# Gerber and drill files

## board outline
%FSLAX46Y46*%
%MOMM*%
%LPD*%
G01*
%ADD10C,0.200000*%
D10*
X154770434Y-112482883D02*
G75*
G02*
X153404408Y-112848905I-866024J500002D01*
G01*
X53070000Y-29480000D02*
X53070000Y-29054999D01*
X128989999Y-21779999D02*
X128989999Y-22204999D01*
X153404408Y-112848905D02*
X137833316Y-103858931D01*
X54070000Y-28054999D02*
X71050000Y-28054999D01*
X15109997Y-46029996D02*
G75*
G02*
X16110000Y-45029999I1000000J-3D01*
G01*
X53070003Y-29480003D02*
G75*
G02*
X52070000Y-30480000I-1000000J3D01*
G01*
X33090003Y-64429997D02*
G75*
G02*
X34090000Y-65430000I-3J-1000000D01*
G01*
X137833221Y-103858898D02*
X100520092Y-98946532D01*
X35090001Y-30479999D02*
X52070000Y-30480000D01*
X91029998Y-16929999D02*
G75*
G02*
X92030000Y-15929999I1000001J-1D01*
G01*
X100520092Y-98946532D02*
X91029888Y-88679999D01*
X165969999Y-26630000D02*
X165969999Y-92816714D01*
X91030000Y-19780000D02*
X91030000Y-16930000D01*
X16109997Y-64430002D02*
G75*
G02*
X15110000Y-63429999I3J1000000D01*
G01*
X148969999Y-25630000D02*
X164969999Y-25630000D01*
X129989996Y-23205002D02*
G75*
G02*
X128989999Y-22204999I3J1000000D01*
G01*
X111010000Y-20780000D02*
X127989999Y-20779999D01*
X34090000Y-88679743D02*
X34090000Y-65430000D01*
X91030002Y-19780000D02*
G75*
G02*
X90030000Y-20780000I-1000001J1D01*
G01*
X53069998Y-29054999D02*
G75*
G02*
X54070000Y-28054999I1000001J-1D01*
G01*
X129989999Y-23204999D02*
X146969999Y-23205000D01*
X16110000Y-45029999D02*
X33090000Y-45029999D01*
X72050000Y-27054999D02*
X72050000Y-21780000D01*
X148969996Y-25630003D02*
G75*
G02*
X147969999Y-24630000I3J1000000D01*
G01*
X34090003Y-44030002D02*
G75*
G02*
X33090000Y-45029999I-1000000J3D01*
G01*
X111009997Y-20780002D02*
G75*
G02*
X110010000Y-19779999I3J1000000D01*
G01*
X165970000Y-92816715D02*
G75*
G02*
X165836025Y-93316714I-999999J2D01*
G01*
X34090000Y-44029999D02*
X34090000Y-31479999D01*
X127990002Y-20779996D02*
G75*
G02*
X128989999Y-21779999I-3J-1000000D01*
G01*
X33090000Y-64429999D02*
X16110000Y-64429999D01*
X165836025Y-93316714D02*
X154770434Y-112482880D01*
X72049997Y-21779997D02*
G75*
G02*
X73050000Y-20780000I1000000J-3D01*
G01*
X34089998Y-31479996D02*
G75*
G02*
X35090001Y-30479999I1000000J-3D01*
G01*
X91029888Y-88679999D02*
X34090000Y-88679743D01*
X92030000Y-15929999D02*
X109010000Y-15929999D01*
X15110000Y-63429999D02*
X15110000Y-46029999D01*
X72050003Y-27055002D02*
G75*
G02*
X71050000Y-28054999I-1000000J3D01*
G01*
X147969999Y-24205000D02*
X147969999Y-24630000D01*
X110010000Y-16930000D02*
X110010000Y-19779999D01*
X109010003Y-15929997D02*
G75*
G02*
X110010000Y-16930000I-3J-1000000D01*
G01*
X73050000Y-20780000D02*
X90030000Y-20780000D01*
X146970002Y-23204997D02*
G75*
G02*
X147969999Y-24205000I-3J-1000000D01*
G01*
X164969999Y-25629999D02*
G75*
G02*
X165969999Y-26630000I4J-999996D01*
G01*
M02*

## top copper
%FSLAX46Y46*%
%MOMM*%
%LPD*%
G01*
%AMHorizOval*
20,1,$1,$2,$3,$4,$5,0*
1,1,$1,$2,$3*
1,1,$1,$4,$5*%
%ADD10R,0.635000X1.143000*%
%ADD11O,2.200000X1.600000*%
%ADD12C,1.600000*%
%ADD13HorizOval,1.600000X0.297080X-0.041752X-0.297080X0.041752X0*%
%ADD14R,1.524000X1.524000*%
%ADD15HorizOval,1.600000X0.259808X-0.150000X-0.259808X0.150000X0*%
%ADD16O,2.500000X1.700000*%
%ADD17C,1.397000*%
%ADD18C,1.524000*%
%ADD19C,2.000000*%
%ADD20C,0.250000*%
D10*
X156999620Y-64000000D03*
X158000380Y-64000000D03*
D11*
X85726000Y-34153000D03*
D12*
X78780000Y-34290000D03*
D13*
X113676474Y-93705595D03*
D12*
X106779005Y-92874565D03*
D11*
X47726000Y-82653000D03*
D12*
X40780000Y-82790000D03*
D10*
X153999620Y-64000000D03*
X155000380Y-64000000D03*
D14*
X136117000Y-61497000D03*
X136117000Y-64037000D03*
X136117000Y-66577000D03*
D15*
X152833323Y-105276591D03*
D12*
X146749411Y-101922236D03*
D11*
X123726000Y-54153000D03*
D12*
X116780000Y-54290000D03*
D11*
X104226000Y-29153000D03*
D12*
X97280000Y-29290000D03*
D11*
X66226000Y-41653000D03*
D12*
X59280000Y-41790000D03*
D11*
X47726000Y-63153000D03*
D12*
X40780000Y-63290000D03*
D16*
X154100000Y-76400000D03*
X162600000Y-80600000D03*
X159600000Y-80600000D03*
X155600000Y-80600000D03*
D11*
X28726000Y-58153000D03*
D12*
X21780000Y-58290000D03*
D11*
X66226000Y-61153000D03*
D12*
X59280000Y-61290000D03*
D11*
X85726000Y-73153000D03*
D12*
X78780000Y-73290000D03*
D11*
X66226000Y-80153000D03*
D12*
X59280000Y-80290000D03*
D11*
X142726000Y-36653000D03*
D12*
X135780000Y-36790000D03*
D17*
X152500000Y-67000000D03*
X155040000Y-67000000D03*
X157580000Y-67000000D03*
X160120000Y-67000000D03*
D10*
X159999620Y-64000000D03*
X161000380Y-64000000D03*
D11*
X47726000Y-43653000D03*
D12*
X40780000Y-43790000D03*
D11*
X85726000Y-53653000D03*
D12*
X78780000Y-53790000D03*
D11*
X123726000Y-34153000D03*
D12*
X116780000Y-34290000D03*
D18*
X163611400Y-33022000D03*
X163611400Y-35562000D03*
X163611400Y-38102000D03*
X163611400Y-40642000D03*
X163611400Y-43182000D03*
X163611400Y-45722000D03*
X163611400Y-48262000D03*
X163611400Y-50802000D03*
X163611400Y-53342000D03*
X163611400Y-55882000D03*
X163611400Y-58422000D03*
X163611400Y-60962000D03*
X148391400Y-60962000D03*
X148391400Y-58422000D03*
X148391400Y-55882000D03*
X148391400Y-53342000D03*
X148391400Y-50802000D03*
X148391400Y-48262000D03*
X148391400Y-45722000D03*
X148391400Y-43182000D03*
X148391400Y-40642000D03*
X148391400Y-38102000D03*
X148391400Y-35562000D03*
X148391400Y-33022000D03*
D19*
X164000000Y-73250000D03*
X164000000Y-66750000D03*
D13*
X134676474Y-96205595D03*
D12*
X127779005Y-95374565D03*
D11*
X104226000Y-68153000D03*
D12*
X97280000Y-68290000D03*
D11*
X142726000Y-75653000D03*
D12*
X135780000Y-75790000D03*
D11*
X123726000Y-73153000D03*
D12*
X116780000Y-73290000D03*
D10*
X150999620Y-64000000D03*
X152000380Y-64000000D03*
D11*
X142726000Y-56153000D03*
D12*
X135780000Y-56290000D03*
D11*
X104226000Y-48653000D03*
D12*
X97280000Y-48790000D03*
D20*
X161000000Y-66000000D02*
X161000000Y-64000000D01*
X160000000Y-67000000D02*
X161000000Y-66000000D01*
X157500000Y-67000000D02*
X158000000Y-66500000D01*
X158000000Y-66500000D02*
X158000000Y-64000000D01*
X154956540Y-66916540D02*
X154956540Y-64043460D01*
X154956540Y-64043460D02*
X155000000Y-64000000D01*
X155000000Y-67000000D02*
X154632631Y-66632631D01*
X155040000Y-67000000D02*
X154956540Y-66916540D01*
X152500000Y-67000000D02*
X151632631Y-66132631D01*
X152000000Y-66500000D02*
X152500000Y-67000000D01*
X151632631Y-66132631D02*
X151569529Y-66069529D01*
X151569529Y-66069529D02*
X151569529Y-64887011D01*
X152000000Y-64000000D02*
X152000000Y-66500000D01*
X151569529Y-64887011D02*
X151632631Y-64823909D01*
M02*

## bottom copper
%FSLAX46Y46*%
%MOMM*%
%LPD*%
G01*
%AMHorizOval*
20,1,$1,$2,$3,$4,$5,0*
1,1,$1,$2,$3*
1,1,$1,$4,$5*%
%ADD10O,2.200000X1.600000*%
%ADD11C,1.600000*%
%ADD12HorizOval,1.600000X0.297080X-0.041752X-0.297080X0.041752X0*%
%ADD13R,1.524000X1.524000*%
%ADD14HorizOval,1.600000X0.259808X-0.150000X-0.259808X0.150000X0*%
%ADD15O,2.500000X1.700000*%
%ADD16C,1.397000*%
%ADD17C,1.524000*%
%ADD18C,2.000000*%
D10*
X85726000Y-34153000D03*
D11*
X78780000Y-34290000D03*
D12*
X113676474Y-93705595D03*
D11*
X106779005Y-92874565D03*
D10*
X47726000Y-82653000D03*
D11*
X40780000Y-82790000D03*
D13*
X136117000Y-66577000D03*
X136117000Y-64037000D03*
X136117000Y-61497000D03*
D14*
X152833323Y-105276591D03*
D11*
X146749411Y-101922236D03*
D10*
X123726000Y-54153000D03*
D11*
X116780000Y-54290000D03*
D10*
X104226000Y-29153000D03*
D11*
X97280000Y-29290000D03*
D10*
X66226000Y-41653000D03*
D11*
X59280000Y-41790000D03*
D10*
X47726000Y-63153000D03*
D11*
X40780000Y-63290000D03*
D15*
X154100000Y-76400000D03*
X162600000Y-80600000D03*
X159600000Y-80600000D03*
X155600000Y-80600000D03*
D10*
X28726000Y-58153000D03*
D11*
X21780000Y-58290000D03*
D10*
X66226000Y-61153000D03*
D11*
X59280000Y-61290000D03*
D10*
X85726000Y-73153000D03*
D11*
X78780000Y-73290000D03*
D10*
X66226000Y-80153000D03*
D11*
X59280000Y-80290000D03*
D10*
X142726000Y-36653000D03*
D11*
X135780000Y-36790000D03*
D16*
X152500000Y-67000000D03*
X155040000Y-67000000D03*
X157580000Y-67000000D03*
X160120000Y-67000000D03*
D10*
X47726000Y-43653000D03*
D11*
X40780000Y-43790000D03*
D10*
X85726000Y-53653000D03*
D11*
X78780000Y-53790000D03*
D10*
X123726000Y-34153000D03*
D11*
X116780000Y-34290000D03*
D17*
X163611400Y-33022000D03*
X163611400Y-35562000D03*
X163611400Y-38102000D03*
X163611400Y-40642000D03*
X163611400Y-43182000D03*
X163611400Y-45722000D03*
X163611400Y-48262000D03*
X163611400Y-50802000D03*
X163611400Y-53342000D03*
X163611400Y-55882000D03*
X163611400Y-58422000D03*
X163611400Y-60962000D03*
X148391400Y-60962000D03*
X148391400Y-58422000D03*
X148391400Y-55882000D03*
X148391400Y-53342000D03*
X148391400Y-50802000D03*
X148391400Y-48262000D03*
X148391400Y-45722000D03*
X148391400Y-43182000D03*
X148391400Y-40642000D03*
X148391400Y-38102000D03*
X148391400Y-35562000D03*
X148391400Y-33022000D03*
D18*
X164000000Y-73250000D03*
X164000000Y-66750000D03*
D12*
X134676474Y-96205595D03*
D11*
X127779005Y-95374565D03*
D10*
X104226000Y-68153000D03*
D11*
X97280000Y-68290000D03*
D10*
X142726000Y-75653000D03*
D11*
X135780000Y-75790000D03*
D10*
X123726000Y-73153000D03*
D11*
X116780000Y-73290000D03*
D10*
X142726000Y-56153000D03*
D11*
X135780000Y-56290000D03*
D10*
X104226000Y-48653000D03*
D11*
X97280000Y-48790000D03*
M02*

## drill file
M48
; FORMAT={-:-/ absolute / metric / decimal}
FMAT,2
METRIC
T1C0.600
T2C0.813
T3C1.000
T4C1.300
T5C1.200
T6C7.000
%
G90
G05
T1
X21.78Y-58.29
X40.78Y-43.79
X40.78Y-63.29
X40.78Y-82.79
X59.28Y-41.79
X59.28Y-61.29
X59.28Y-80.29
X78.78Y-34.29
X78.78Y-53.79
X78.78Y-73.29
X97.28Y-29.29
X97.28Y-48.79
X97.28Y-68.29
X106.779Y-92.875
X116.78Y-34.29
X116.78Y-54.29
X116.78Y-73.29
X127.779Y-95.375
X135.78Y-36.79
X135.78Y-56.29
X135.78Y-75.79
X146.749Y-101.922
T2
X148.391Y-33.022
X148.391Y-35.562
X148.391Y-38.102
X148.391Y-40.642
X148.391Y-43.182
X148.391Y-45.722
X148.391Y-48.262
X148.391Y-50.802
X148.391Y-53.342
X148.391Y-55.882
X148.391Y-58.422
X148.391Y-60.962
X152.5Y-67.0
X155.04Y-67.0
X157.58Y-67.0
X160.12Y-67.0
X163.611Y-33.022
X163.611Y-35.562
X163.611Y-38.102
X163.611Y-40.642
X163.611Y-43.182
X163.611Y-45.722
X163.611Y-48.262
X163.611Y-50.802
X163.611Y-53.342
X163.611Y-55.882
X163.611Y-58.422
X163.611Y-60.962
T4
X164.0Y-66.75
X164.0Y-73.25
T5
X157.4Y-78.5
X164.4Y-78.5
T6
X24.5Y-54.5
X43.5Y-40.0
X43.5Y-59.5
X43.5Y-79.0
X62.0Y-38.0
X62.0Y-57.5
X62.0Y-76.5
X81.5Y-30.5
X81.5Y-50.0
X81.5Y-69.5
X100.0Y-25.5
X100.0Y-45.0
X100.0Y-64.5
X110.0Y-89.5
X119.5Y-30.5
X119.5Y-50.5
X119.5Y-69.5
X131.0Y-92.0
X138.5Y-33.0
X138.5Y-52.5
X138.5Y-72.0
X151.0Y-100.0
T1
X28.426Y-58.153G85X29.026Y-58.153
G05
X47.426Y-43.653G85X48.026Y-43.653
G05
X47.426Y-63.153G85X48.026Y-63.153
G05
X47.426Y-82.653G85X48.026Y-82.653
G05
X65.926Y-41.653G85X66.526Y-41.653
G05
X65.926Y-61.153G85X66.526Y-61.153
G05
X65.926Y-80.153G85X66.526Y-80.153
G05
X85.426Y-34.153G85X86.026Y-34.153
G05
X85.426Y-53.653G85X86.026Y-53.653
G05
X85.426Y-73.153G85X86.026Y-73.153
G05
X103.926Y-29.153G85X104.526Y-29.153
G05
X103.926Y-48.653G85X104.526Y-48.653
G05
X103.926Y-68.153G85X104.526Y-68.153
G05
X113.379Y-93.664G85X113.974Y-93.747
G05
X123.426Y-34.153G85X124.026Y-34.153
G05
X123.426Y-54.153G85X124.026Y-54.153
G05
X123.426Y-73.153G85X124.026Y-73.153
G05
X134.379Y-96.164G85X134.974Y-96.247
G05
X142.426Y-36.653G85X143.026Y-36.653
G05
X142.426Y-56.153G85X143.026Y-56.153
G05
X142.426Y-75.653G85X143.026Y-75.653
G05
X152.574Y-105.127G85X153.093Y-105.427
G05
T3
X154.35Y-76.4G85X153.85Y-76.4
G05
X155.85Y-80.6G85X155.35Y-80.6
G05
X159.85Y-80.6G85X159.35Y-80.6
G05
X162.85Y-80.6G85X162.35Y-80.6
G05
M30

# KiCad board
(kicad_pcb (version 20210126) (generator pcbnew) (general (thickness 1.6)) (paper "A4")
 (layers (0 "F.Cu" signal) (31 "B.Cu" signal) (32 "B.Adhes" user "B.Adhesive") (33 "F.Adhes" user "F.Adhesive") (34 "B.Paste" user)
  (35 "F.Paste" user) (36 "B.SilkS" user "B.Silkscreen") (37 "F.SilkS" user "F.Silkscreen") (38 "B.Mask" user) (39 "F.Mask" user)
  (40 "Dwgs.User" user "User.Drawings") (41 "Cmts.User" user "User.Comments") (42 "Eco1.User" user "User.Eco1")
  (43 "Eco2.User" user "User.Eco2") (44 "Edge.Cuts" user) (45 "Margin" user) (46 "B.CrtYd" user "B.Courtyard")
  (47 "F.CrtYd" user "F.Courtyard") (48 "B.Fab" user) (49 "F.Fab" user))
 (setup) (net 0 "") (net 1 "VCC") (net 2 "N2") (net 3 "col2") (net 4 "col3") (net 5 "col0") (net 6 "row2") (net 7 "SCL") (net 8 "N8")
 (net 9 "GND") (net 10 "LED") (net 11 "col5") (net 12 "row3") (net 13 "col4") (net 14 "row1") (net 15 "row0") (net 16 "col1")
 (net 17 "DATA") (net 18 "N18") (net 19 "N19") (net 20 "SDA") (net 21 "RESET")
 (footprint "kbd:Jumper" (layer "F.Cu") (at 157.5 64)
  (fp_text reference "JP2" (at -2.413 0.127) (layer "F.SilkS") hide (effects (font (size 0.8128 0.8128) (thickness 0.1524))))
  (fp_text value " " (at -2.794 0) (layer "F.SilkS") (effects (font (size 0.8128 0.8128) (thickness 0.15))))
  (pad "1" smd rect (at -0.50038 0) (locked) (size 0.635 1.143) (layers "F.Cu" "F.Paste" "F.Mask") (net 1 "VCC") (clearance 0.1905))
  (pad "2" smd rect (at 0.50038 0) (locked) (size 0.635 1.143) (layers "F.Cu" "F.Paste" "F.Mask") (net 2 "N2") (clearance 0.1905)))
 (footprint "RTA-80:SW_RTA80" (layer "F.Cu") (at 81.5 30.5)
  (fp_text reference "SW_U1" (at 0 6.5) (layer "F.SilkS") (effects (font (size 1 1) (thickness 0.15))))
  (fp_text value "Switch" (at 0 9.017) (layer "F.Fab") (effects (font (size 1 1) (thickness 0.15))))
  (pad "" np_thru_hole circle (at 0 0) (locked) (size 7 7) (drill 7) (layers *.Cu *.Mask))
  (pad "1" thru_hole oval (at 4.226 3.653) (locked) (size 2.2 1.6) (drill oval 1.2 0.6) (layers *.Cu *.Mask) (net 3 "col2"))
  (pad "2" thru_hole circle (at -2.72 3.79) (locked) (size 1.6 1.6) (drill 0.6) (layers *.Cu *.Mask)))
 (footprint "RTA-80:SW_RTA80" (layer "F.Cu") (at 110 89.5 -8)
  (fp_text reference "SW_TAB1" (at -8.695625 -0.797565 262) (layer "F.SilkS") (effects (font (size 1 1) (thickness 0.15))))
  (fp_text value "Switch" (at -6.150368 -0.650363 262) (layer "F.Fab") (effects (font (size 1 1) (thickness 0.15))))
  (pad "" np_thru_hole circle (at 0 0 352) (locked) (size 7 7) (drill 7) (layers *.Cu *.Mask))
  (pad "1" thru_hole oval (at 4.226 3.653 352) (locked) (size 2.2 1.6) (drill oval 1.2 0.6) (layers *.Cu *.Mask) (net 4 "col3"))
  (pad "2" thru_hole circle (at -2.72 3.79 352) (locked) (size 1.6 1.6) (drill 0.6) (layers *.Cu *.Mask)))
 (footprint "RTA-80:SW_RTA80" (layer "F.Cu") (at 43.5 79)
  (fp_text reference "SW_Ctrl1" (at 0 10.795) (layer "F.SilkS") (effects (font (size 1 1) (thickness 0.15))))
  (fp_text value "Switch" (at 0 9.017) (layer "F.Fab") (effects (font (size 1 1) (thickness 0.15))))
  (pad "" np_thru_hole circle (at 0 0) (locked) (size 7 7) (drill 7) (layers *.Cu *.Mask))
  (pad "1" thru_hole oval (at 4.226 3.653) (locked) (size 2.2 1.6) (drill oval 1.2 0.6) (layers *.Cu *.Mask) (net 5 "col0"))
  (pad "2" thru_hole circle (at -2.72 3.79) (locked) (size 1.6 1.6) (drill 0.6) (layers *.Cu *.Mask) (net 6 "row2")))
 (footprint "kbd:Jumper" (layer "F.Cu") (at 154.5 64)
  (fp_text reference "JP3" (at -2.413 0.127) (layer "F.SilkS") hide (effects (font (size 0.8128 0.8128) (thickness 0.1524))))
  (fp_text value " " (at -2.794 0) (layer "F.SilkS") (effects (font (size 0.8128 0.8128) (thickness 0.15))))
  (pad "1" smd rect (at -0.50038 0) (locked) (size 0.635 1.143) (layers "F.Cu" "F.Paste" "F.Mask") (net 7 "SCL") (clearance 0.1905))
  (pad "2" smd rect (at 0.50038 0) (locked) (size 0.635 1.143) (layers "F.Cu" "F.Paste" "F.Mask") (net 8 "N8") (clearance 0.1905)))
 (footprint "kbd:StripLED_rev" (layer "F.Cu") (at 136.117 61.497)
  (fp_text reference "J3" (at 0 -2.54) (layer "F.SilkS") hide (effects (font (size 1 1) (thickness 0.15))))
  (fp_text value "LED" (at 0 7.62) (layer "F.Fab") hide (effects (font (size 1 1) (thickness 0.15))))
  (pad "1" smd rect (at 0 0) (locked) (size 1.524 1.524) (layers "F.Cu" "F.Paste" "F.Mask") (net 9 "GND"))
  (pad "1" smd rect (at 0 5.08) (locked) (size 1.524 1.524) (layers "B.Cu" "B.Paste" "B.Mask") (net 9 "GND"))
  (pad "2" smd rect (at 0 2.54) (locked) (size 1.524 1.524) (layers "B.Cu" "B.Paste" "B.Mask") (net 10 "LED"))
  (pad "2" smd rect (at 0 2.54) (locked) (size 1.524 1.524) (layers "F.Cu" "F.Paste" "F.Mask") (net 10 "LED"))
  (pad "3" smd rect (at 0 0) (locked) (size 1.524 1.524) (layers "B.Cu" "B.Paste" "B.Mask") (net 1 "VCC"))
  (pad "3" smd rect (at 0 5.08) (locked) (size 1.524 1.524) (layers "F.Cu" "F.Paste" "F.Mask") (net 1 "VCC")))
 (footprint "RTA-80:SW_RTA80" (layer "F.Cu") (at 151 100 -30)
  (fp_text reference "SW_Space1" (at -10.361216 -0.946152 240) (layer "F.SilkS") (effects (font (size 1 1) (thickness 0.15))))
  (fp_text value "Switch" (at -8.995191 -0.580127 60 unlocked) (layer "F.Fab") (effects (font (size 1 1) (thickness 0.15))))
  (pad "" np_thru_hole circle (at 0 0 330) (locked) (size 7 7) (drill 7) (layers *.Cu *.Mask))
  (pad "1" thru_hole oval (at 4.226 3.653 330) (locked) (size 2.2 1.6) (drill oval 1.2 0.6) (layers *.Cu *.Mask) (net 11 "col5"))
  (pad "2" thru_hole circle (at -2.72 3.79 330) (locked) (size 1.6 1.6) (drill 0.6) (layers *.Cu *.Mask) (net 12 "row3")))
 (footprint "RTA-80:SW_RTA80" (layer "F.Cu") (at 119.5 50.5)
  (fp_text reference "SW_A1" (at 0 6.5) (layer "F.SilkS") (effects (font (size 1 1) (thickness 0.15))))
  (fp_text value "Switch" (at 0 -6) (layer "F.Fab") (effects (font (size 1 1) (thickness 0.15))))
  (pad "" np_thru_hole circle (at 0 0) (locked) (size 7 7) (drill 7) (layers *.Cu *.Mask))
  (pad "1" thru_hole oval (at 4.226 3.653) (locked) (size 2.2 1.6) (drill oval 1.2 0.6) (layers *.Cu *.Mask) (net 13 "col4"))
  (pad "2" thru_hole circle (at -2.72 3.79) (locked) (size 1.6 1.6) (drill 0.6) (layers *.Cu *.Mask) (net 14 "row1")))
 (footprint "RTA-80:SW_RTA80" (layer "F.Cu") (at 100 25.5)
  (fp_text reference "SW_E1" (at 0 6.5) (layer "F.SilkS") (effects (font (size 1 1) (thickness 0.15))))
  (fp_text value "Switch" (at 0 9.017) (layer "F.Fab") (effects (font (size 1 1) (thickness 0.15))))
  (pad "" np_thru_hole circle (at 0 0) (locked) (size 7 7) (drill 7) (layers *.Cu *.Mask))
  (pad "1" thru_hole oval (at 4.226 3.653) (locked) (size 2.2 1.6) (drill oval 1.2 0.6) (layers *.Cu *.Mask) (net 4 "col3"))
  (pad "2" thru_hole circle (at -2.72 3.79) (locked) (size 1.6 1.6) (drill 0.6) (layers *.Cu *.Mask) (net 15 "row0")))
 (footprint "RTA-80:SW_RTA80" (layer "F.Cu") (at 62 38)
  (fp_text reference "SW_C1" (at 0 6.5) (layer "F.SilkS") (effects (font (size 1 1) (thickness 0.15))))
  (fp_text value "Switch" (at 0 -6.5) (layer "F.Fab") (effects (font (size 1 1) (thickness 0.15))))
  (pad "" np_thru_hole circle (at 0 0) (locked) (size 7 7) (drill 7) (layers *.Cu *.Mask))
  (pad "1" thru_hole oval (at 4.226 3.653) (locked) (size 2.2 1.6) (drill oval 1.2 0.6) (layers *.Cu *.Mask) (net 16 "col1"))
  (pad "2" thru_hole circle (at -2.72 3.79) (locked) (size 1.6 1.6) (drill 0.6) (layers *.Cu *.Mask) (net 15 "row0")))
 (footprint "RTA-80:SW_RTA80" (layer "F.Cu") (at 43.5 59.5)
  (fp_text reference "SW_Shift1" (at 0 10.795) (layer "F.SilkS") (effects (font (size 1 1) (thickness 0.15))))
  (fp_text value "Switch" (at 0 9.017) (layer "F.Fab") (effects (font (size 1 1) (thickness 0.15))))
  (pad "" np_thru_hole circle (at 0 0) (locked) (size 7 7) (drill 7) (layers *.Cu *.Mask))
  (pad "1" thru_hole oval (at 4.226 3.653) (locked) (size 2.2 1.6) (drill oval 1.2 0.6) (layers *.Cu *.Mask) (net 5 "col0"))
  (pad "2" thru_hole circle (at -2.72 3.79) (locked) (size 1.6 1.6) (drill 0.6) (layers *.Cu *.Mask) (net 14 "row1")))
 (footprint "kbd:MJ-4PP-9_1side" (layer "F.Cu") (at 165.9 78.5 -90)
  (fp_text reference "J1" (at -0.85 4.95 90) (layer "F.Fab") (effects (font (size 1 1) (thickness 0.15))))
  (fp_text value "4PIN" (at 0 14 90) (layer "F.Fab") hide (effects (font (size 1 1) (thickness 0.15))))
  (pad "" np_thru_hole circle (at 0 8.5 270) (locked) (size 1.2 1.2) (drill 1.2) (layers *.Cu *.Mask))
  (pad "" np_thru_hole circle (at 0 1.5 270) (locked) (size 1.2 1.2) (drill 1.2) (layers *.Cu *.Mask))
  (pad "A" thru_hole oval (at -2.1 11.8 270) (locked) (size 1.7 2.5) (drill oval 1 1.5) (layers *.Cu "B.Mask") (clearance 0.15))
  (pad "B" thru_hole oval (at 2.1 3.3 270) (locked) (size 1.7 2.5) (drill oval 1 1.5) (layers *.Cu "B.Mask") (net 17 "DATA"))
  (pad "C" thru_hole oval (at 2.1 6.3 270) (locked) (size 1.7 2.5) (drill oval 1 1.5) (layers *.Cu "B.Mask") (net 9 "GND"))
  (pad "D" thru_hole oval (at 2.1 10.3 270) (locked) (size 1.7 2.5) (drill oval 1 1.5) (layers *.Cu "B.Mask") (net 1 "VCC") (clearance 0.15)))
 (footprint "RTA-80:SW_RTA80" (layer "F.Cu") (at 24.5 54.5)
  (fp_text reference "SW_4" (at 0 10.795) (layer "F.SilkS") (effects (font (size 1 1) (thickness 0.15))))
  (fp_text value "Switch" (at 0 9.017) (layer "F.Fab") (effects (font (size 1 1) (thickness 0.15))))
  (pad "" np_thru_hole circle (at 0 0) (locked) (size 7 7) (drill 7) (layers *.Cu *.Mask))
  (pad "1" thru_hole oval (at 4.226 3.653) (locked) (size 2.2 1.6) (drill oval 1.2 0.6) (layers *.Cu *.Mask) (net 5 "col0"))
  (pad "2" thru_hole circle (at -2.72 3.79) (locked) (size 1.6 1.6) (drill 0.6) (layers *.Cu *.Mask) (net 12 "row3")))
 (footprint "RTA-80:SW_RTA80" (layer "F.Cu") (at 62 57.5)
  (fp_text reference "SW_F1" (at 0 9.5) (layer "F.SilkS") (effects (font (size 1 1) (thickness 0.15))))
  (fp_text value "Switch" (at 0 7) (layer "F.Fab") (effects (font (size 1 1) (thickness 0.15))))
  (pad "" np_thru_hole circle (at 0 0) (locked) (size 7 7) (drill 7) (layers *.Cu *.Mask))
  (pad "1" thru_hole oval (at 4.226 3.653) (locked) (size 2.2 1.6) (drill oval 1.2 0.6) (layers *.Cu *.Mask) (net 16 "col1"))
  (pad "2" thru_hole circle (at -2.72 3.79) (locked) (size 1.6 1.6) (drill 0.6) (layers *.Cu *.Mask) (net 14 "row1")))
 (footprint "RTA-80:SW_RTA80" (layer "F.Cu") (at 81.5 69.5)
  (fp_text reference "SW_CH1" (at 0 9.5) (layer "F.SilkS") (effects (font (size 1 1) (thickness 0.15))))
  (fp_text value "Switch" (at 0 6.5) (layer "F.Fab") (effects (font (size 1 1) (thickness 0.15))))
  (pad "" np_thru_hole circle (at 0 0) (locked) (size 7 7) (drill 7) (layers *.Cu *.Mask))
  (pad "1" thru_hole oval (at 4.226 3.653) (locked) (size 2.2 1.6) (drill oval 1.2 0.6) (layers *.Cu *.Mask) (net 3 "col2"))
  (pad "2" thru_hole circle (at -2.72 3.79) (locked) (size 1.6 1.6) (drill 0.6) (layers *.Cu *.Mask) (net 6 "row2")))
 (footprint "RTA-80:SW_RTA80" (layer "F.Cu") (at 62 76.5)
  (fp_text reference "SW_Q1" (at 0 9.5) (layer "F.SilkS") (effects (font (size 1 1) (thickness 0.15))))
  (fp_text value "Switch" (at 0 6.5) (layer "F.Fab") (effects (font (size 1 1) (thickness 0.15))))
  (pad "" np_thru_hole circle (at 0 0) (locked) (size 7 7) (drill 7) (layers *.Cu *.Mask))
  (pad "1" thru_hole oval (at 4.226 3.653) (locked) (size 2.2 1.6) (drill oval 1.2 0.6) (layers *.Cu *.Mask) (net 16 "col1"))
  (pad "2" thru_hole circle (at -2.72 3.79) (locked) (size 1.6 1.6) (drill 0.6) (layers *.Cu *.Mask) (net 6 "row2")))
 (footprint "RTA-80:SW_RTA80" (layer "F.Cu") (at 138.5 33)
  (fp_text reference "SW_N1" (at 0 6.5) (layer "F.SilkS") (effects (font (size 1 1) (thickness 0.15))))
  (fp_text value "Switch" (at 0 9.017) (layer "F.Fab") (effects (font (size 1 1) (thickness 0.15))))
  (pad "" np_thru_hole circle (at 0 0) (locked) (size 7 7) (drill 7) (layers *.Cu *.Mask))
  (pad "1" thru_hole oval (at 4.226 3.653) (locked) (size 2.2 1.6) (drill oval 1.2 0.6) (layers *.Cu *.Mask) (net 11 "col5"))
  (pad "2" thru_hole circle (at -2.72 3.79) (locked) (size 1.6 1.6) (drill 0.6) (layers *.Cu *.Mask) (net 15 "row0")))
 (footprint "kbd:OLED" (layer "F.Cu") (at 152.5 67)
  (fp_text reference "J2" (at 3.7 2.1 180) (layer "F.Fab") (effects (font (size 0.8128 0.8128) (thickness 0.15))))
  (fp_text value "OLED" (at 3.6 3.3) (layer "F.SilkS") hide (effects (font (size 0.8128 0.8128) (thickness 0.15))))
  (pad "1" thru_hole circle (at 0 0) (locked) (size 1.397 1.397) (drill 0.8128) (layers *.Cu *.Mask "F.SilkS") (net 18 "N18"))
  (pad "2" thru_hole circle (at 2.54 0) (locked) (size 1.397 1.397) (drill 0.8128) (layers *.Cu *.Mask "F.SilkS") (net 8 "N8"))
  (pad "3" thru_hole circle (at 5.08 0) (locked) (size 1.397 1.397) (drill 0.8128) (layers *.Cu *.Mask "F.SilkS") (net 2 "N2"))
  (pad "4" thru_hole circle (at 7.62 0) (locked) (size 1.397 1.397) (drill 0.8128) (layers *.Cu *.Mask "F.SilkS") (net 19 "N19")))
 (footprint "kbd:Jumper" (layer "F.Cu") (at 160.5 64)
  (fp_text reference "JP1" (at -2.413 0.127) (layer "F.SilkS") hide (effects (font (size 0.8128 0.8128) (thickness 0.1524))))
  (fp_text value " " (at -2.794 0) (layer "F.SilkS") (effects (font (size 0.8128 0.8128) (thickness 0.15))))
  (pad "1" smd rect (at -0.50038 0) (locked) (size 0.635 1.143) (layers "F.Cu" "F.Paste" "F.Mask") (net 9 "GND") (clearance 0.1905))
  (pad "2" smd rect (at 0.50038 0) (locked) (size 0.635 1.143) (layers "F.Cu" "F.Paste" "F.Mask") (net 19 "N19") (clearance 0.1905)))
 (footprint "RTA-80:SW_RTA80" (layer "F.Cu") (at 43.5 40)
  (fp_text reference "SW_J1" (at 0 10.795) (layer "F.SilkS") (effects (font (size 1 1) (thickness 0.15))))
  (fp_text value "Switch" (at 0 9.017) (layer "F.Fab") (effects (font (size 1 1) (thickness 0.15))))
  (pad "" np_thru_hole circle (at 0 0) (locked) (size 7 7) (drill 7) (layers *.Cu *.Mask))
  (pad "1" thru_hole oval (at 4.226 3.653) (locked) (size 2.2 1.6) (drill oval 1.2 0.6) (layers *.Cu *.Mask) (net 5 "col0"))
  (pad "2" thru_hole circle (at -2.72 3.79) (locked) (size 1.6 1.6) (drill 0.6) (layers *.Cu *.Mask) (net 15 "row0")))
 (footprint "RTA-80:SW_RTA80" (layer "F.Cu") (at 81.5 50)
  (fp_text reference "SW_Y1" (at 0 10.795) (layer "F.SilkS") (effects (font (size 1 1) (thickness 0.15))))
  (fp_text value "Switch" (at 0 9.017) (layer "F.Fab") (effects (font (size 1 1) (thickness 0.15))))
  (pad "" np_thru_hole circle (at 0 0) (locked) (size 7 7) (drill 7) (layers *.Cu *.Mask))
  (pad "1" thru_hole oval (at 4.226 3.653) (locked) (size 2.2 1.6) (drill oval 1.2 0.6) (layers *.Cu *.Mask) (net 3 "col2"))
  (pad "2" thru_hole circle (at -2.72 3.79) (locked) (size 1.6 1.6) (drill 0.6) (layers *.Cu *.Mask) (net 14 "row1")))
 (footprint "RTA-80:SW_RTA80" (layer "F.Cu") (at 119.5 30.5)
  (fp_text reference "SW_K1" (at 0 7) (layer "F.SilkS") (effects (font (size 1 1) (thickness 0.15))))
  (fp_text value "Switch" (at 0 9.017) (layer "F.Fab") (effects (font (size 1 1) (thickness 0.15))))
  (pad "" np_thru_hole circle (at 0 0) (locked) (size 7 7) (drill 7) (layers *.Cu *.Mask))
  (pad "1" thru_hole oval (at 4.226 3.653) (locked) (size 2.2 1.6) (drill oval 1.2 0.6) (layers *.Cu *.Mask) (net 13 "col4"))
  (pad "2" thru_hole circle (at -2.72 3.79) (locked) (size 1.6 1.6) (drill 0.6) (layers *.Cu *.Mask)))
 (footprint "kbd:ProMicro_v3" (layer "F.Cu") (at 156 47.5)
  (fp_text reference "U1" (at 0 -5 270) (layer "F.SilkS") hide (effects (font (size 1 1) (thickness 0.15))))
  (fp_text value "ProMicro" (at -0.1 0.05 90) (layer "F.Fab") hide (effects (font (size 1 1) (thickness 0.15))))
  (pad "1" thru_hole circle (at 7.6114 -14.478) (locked) (size 1.524 1.524) (drill 0.8128) (layers *.Cu "B.Mask") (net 10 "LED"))
  (pad "2" thru_hole circle (at 7.6114 -11.938) (locked) (size 1.524 1.524) (drill 0.8128) (layers *.Cu "B.Mask") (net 17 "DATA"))
  (pad "3" thru_hole circle (at 7.6114 -9.398) (locked) (size 1.524 1.524) (drill 0.8128) (layers *.Cu "B.Mask") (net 9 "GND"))
  (pad "4" thru_hole circle (at 7.6114 -6.858) (locked) (size 1.524 1.524) (drill 0.8128) (layers *.Cu "B.Mask") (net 9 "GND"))
  (pad "5" thru_hole circle (at 7.6114 -4.318) (locked) (size 1.524 1.524) (drill 0.8128) (layers *.Cu "B.Mask") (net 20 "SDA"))
  (pad "6" thru_hole circle (at 7.6114 -1.778) (locked) (size 1.524 1.524) (drill 0.8128) (layers *.Cu "B.Mask") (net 7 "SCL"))
  (pad "7" thru_hole circle (at 7.6114 0.762) (locked) (size 1.524 1.524) (drill 0.8128) (layers *.Cu "B.Mask"))
  (pad "8" thru_hole circle (at 7.6114 3.302) (locked) (size 1.524 1.524) (drill 0.8128) (layers *.Cu "B.Mask") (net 15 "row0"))
  (pad "9" thru_hole circle (at 7.6114 5.842) (locked) (size 1.524 1.524) (drill 0.8128) (layers *.Cu "B.Mask") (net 14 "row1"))
  (pad "10" thru_hole circle (at 7.6114 8.382) (locked) (size 1.524 1.524) (drill 0.8128) (layers *.Cu "B.Mask") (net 6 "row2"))
  (pad "11" thru_hole circle (at 7.6114 10.922) (locked) (size 1.524 1.524) (drill 0.8128) (layers *.Cu "B.Mask") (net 12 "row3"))
  (pad "12" thru_hole circle (at 7.6114 13.462) (locked) (size 1.524 1.524) (drill 0.8128) (layers *.Cu "B.Mask"))
  (pad "13" thru_hole circle (at -7.6086 13.462) (locked) (size 1.524 1.524) (drill 0.8128) (layers *.Cu "B.Mask") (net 11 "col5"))
  (pad "14" thru_hole circle (at -7.6086 10.922) (locked) (size 1.524 1.524) (drill 0.8128) (layers *.Cu "B.Mask") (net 13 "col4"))
  (pad "15" thru_hole circle (at -7.6086 8.382) (locked) (size 1.524 1.524) (drill 0.8128) (layers *.Cu "B.Mask") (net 4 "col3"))
  (pad "16" thru_hole circle (at -7.6086 5.842) (locked) (size 1.524 1.524) (drill 0.8128) (layers *.Cu "B.Mask") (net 3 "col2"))
  (pad "17" thru_hole circle (at -7.6086 3.302) (locked) (size 1.524 1.524) (drill 0.8128) (layers *.Cu "B.Mask") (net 16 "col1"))
  (pad "18" thru_hole circle (at -7.6086 0.762) (locked) (size 1.524 1.524) (drill 0.8128) (layers *.Cu "B.Mask") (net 5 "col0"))
  (pad "19" thru_hole circle (at -7.6086 -1.778) (locked) (size 1.524 1.524) (drill 0.8128) (layers *.Cu "B.Mask"))
  (pad "20" thru_hole circle (at -7.6086 -4.318) (locked) (size 1.524 1.524) (drill 0.8128) (layers *.Cu "B.Mask"))
  (pad "21" thru_hole circle (at -7.6086 -6.858) (locked) (size 1.524 1.524) (drill 0.8128) (layers *.Cu "B.Mask") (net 1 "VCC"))
  (pad "22" thru_hole circle (at -7.6086 -9.398) (locked) (size 1.524 1.524) (drill 0.8128) (layers *.Cu "B.Mask") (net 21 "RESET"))
  (pad "23" thru_hole circle (at -7.6086 -11.938) (locked) (size 1.524 1.524) (drill 0.8128) (layers *.Cu "B.Mask") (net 9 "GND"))
  (pad "24" thru_hole circle (at -7.6086 -14.478) (locked) (size 1.524 1.524) (drill 0.8128) (layers *.Cu "B.Mask")))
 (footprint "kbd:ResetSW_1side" (layer "F.Cu") (at 164 70 -90)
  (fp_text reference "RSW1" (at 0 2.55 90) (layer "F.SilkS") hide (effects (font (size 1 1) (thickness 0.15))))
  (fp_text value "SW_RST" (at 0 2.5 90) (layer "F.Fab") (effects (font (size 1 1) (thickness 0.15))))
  (pad "1" thru_hole circle (at 3.25 0 270) (locked) (size 2 2) (drill 1.3) (layers *.Cu "B.Mask") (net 9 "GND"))
  (pad "2" thru_hole circle (at -3.25 0 270) (locked) (size 2 2) (drill 1.3) (layers *.Cu "B.Mask") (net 21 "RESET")))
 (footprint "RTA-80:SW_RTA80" (layer "F.Cu") (at 131 92 -8)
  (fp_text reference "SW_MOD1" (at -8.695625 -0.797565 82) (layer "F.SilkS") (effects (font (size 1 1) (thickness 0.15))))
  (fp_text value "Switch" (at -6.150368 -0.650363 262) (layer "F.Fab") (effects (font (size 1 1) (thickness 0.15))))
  (pad "" np_thru_hole circle (at 0 0 352) (locked) (size 7 7) (drill 7) (layers *.Cu *.Mask))
  (pad "1" thru_hole oval (at 4.226 3.653 352) (locked) (size 2.2 1.6) (drill oval 1.2 0.6) (layers *.Cu *.Mask) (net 13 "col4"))
  (pad "2" thru_hole circle (at -2.72 3.79 352) (locked) (size 1.6 1.6) (drill 0.6) (layers *.Cu *.Mask) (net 12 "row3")))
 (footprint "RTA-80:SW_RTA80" (layer "F.Cu") (at 100 64.5)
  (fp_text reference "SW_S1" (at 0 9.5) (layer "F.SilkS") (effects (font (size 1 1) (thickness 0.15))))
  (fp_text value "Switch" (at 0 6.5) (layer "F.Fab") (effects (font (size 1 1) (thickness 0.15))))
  (pad "" np_thru_hole circle (at 0 0) (locked) (size 7 7) (drill 7) (layers *.Cu *.Mask))
  (pad "1" thru_hole oval (at 4.226 3.653) (locked) (size 2.2 1.6) (drill oval 1.2 0.6) (layers *.Cu *.Mask) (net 4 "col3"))
  (pad "2" thru_hole circle (at -2.72 3.79) (locked) (size 1.6 1.6) (drill 0.6) (layers *.Cu *.Mask)))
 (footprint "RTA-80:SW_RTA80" (layer "F.Cu") (at 138.5 72)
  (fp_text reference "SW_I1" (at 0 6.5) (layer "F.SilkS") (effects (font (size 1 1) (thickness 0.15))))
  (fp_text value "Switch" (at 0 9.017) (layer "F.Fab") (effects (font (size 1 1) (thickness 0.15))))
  (pad "" np_thru_hole circle (at 0 0) (locked) (size 7 7) (drill 7) (layers *.Cu *.Mask))
  (pad "1" thru_hole oval (at 4.226 3.653) (locked) (size 2.2 1.6) (drill oval 1.2 0.6) (layers *.Cu *.Mask) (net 11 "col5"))
  (pad "2" thru_hole circle (at -2.72 3.79) (locked) (size 1.6 1.6) (drill 0.6) (layers *.Cu *.Mask) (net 6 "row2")))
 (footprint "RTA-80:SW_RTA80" (layer "F.Cu") (at 119.5 69.5)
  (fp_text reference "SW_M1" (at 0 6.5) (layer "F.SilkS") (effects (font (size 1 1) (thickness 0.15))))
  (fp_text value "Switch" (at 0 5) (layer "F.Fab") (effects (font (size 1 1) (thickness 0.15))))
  (pad "" np_thru_hole circle (at 0 0) (locked) (size 7 7) (drill 7) (layers *.Cu *.Mask))
  (pad "1" thru_hole oval (at 4.226 3.653) (locked) (size 2.2 1.6) (drill oval 1.2 0.6) (layers *.Cu *.Mask) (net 13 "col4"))
  (pad "2" thru_hole circle (at -2.72 3.79) (locked) (size 1.6 1.6) (drill 0.6) (layers *.Cu *.Mask) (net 6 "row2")))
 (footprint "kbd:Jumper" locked (layer "F.Cu") (at 151.5 64)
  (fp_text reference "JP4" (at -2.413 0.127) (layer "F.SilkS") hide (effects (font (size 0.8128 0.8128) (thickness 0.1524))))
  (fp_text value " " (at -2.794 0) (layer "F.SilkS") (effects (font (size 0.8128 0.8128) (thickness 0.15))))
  (pad "1" smd rect (at -0.50038 0) (locked) (size 0.635 1.143) (layers "F.Cu" "F.Paste" "F.Mask") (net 20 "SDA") (clearance 0.1905))
  (pad "2" smd rect (at 0.50038 0) (locked) (size 0.635 1.143) (layers "F.Cu" "F.Paste" "F.Mask") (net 18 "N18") (clearance 0.1905)))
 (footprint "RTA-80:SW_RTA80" (layer "F.Cu") (at 138.5 52.5)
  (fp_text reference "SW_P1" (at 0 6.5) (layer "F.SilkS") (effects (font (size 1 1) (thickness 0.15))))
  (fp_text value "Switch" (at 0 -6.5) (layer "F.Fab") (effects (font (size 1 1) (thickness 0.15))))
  (pad "" np_thru_hole circle (at 0 0) (locked) (size 7 7) (drill 7) (layers *.Cu *.Mask))
  (pad "1" thru_hole oval (at 4.226 3.653) (locked) (size 2.2 1.6) (drill oval 1.2 0.6) (layers *.Cu *.Mask) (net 11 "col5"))
  (pad "2" thru_hole circle (at -2.72 3.79) (locked) (size 1.6 1.6) (drill 0.6) (layers *.Cu *.Mask) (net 14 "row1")))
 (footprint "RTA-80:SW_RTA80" (layer "F.Cu") (at 100 45)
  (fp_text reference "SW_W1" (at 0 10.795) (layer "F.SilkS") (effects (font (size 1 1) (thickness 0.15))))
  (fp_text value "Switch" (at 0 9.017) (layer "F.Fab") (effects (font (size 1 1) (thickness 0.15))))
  (pad "" np_thru_hole circle (at 0 0) (locked) (size 7 7) (drill 7) (layers *.Cu *.Mask))
  (pad "1" thru_hole oval (at 4.226 3.653) (locked) (size 2.2 1.6) (drill oval 1.2 0.6) (layers *.Cu *.Mask) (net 4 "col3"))
  (pad "2" thru_hole circle (at -2.72 3.79) (locked) (size 1.6 1.6) (drill 0.6) (layers *.Cu *.Mask)))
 (gr_arc (start 153.90441 111.982881) (end 153.404408 112.848905) (angle -90) (layer "Edge.Cuts") (width 0.2))
 (gr_line (start 53.07 29.48) (end 53.07 29.054999) (layer "Edge.Cuts") (width 0.2))
 (gr_line (start 128.989999 21.779999) (end 128.989999 22.204999) (layer "Edge.Cuts") (width 0.2))
 (gr_line (start 153.404408 112.848905) (end 137.833316 103.858931) (layer "Edge.Cuts") (width 0.2))
 (gr_line (start 54.07 28.054999) (end 71.05 28.054999) (layer "Edge.Cuts") (width 0.2))
 (gr_arc (start 16.109997 46.029999) (end 16.11 45.029999) (angle -90) (layer "Edge.Cuts") (width 0.2))
 (gr_arc (start 52.070003 29.48) (end 52.07 30.48) (angle -90) (layer "Edge.Cuts") (width 0.2))
 (gr_arc (start 33.09 65.429997) (end 34.09 65.43) (angle -90) (layer "Edge.Cuts") (width 0.2))
 (gr_line (start 137.833221 103.858898) (end 100.520092 98.946532) (layer "Edge.Cuts") (width 0.2))
 (gr_line (start 35.090001 30.479999) (end 52.07 30.48) (layer "Edge.Cuts") (width 0.2))
 (gr_arc (start 92.029999 16.93) (end 92.03 15.929999) (angle -90) (layer "Edge.Cuts") (width 0.2))
 (gr_line (start 100.520092 98.946532) (end 91.029888 88.679999) (layer "Edge.Cuts") (width 0.2))
 (gr_line (start 165.969999 26.63) (end 165.969999 92.816714) (layer "Edge.Cuts") (width 0.2))
 (gr_line (start 91.03 19.78) (end 91.03 16.93) (layer "Edge.Cuts") (width 0.2))
 (gr_arc (start 16.11 63.430002) (end 15.11 63.429999) (angle -90) (layer "Edge.Cuts") (width 0.2))
 (gr_line (start 148.969999 25.63) (end 164.969999 25.63) (layer "Edge.Cuts") (width 0.2))
 (gr_arc (start 129.989999 22.205002) (end 128.989999 22.204999) (angle -90) (layer "Edge.Cuts") (width 0.2))
 (gr_line (start 111.01 20.78) (end 127.989999 20.779999) (layer "Edge.Cuts") (width 0.2))
 (gr_line (start 34.09 88.679743) (end 34.09 65.43) (layer "Edge.Cuts") (width 0.2))
 (gr_arc (start 90.030001 19.779999) (end 90.03 20.78) (angle -90) (layer "Edge.Cuts") (width 0.2))
 (gr_arc (start 54.069999 29.055) (end 54.07 28.054999) (angle -90) (layer "Edge.Cuts") (width 0.2))
 (gr_line (start 129.989999 23.204999) (end 146.969999 23.205) (layer "Edge.Cuts") (width 0.2))
 (gr_line (start 16.11 45.029999) (end 33.09 45.029999) (layer "Edge.Cuts") (width 0.2))
 (gr_line (start 72.05 27.054999) (end 72.05 21.78) (layer "Edge.Cuts") (width 0.2))
 (gr_arc (start 148.969999 24.630003) (end 147.969999 24.63) (angle -90) (layer "Edge.Cuts") (width 0.2))
 (gr_arc (start 33.090003 44.029999) (end 33.09 45.029999) (angle -90) (layer "Edge.Cuts") (width 0.2))
 (gr_arc (start 111.01 19.780002) (end 110.01 19.779999) (angle -90) (layer "Edge.Cuts") (width 0.2))
 (gr_arc (start 164.970001 92.816713) (end 165.836025 93.316714) (angle -30) (layer "Edge.Cuts") (width 0.2))
 (gr_line (start 34.09 44.029999) (end 34.09 31.479999) (layer "Edge.Cuts") (width 0.2))
 (gr_arc (start 127.989999 21.779996) (end 128.989999 21.779999) (angle -90) (layer "Edge.Cuts") (width 0.2))
 (gr_line (start 33.09 64.429999) (end 16.11 64.429999) (layer "Edge.Cuts") (width 0.2))
 (gr_line (start 165.836025 93.316714) (end 154.770434 112.48288) (layer "Edge.Cuts") (width 0.2))
 (gr_arc (start 73.049997 21.78) (end 73.05 20.78) (angle -90) (layer "Edge.Cuts") (width 0.2))
 (gr_arc (start 35.089998 31.479999) (end 35.090001 30.479999) (angle -90) (layer "Edge.Cuts") (width 0.2))
 (gr_line (start 91.029888 88.679999) (end 34.09 88.679743) (layer "Edge.Cuts") (width 0.2))
 (gr_line (start 92.03 15.929999) (end 109.01 15.929999) (layer "Edge.Cuts") (width 0.2))
 (gr_line (start 15.11 63.429999) (end 15.11 46.029999) (layer "Edge.Cuts") (width 0.2))
 (gr_arc (start 71.050003 27.054999) (end 71.05 28.054999) (angle -90) (layer "Edge.Cuts") (width 0.2))
 (gr_line (start 147.969999 24.205) (end 147.969999 24.63) (layer "Edge.Cuts") (width 0.2))
 (gr_line (start 110.01 16.93) (end 110.01 19.779999) (layer "Edge.Cuts") (width 0.2))
 (gr_arc (start 109.01 16.929997) (end 110.01 16.93) (angle -90) (layer "Edge.Cuts") (width 0.2))
 (gr_line (start 73.05 20.78) (end 90.03 20.78) (layer "Edge.Cuts") (width 0.2))
 (gr_arc (start 146.969999 24.204997) (end 147.969999 24.205) (angle -90) (layer "Edge.Cuts") (width 0.2))
 (gr_arc (start 164.970003 26.629995) (end 165.969999 26.63) (angle -90.00051566) (layer "Edge.Cuts") (width 0.2))
 (segment (start 161 66) (end 161 64) (width 0.25) (layer "F.Cu") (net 19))
 (segment (start 160 67) (end 161 66) (width 0.25) (layer "F.Cu") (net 19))
 (segment (start 157.5 67) (end 158 66.5) (width 0.25) (layer "F.Cu") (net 2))
 (segment (start 158 66.5) (end 158 64) (width 0.25) (layer "F.Cu") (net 2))
 (segment (start 154.95654 66.91654) (end 154.95654 64.04346) (width 0.25) (layer "F.Cu") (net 8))
 (segment (start 154.95654 64.04346) (end 155 64) (width 0.25) (layer "F.Cu") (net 8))
 (segment (start 155 67) (end 154.632631 66.632631) (width 0.25) (layer "F.Cu") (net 8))
 (segment (start 155.04 67) (end 154.95654 66.91654) (width 0.25) (layer "F.Cu") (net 8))
 (segment (start 152.5 67) (end 151.632631 66.132631) (width 0.25) (layer "F.Cu") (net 18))
 (segment (start 152 66.5) (end 152.5 67) (width 0.25) (layer "F.Cu") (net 18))
 (segment (start 151.632631 66.132631) (end 151.569529 66.069529) (width 0.25) (layer "F.Cu") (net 18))
 (segment (start 151.569529 66.069529) (end 151.569529 64.887011) (width 0.25) (layer "F.Cu") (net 18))
 (segment (start 152 64) (end 152 66.5) (width 0.25) (layer "F.Cu") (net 18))
 (segment (start 151.569529 64.887011) (end 151.632631 64.823909) (width 0.25) (layer "F.Cu") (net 18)))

